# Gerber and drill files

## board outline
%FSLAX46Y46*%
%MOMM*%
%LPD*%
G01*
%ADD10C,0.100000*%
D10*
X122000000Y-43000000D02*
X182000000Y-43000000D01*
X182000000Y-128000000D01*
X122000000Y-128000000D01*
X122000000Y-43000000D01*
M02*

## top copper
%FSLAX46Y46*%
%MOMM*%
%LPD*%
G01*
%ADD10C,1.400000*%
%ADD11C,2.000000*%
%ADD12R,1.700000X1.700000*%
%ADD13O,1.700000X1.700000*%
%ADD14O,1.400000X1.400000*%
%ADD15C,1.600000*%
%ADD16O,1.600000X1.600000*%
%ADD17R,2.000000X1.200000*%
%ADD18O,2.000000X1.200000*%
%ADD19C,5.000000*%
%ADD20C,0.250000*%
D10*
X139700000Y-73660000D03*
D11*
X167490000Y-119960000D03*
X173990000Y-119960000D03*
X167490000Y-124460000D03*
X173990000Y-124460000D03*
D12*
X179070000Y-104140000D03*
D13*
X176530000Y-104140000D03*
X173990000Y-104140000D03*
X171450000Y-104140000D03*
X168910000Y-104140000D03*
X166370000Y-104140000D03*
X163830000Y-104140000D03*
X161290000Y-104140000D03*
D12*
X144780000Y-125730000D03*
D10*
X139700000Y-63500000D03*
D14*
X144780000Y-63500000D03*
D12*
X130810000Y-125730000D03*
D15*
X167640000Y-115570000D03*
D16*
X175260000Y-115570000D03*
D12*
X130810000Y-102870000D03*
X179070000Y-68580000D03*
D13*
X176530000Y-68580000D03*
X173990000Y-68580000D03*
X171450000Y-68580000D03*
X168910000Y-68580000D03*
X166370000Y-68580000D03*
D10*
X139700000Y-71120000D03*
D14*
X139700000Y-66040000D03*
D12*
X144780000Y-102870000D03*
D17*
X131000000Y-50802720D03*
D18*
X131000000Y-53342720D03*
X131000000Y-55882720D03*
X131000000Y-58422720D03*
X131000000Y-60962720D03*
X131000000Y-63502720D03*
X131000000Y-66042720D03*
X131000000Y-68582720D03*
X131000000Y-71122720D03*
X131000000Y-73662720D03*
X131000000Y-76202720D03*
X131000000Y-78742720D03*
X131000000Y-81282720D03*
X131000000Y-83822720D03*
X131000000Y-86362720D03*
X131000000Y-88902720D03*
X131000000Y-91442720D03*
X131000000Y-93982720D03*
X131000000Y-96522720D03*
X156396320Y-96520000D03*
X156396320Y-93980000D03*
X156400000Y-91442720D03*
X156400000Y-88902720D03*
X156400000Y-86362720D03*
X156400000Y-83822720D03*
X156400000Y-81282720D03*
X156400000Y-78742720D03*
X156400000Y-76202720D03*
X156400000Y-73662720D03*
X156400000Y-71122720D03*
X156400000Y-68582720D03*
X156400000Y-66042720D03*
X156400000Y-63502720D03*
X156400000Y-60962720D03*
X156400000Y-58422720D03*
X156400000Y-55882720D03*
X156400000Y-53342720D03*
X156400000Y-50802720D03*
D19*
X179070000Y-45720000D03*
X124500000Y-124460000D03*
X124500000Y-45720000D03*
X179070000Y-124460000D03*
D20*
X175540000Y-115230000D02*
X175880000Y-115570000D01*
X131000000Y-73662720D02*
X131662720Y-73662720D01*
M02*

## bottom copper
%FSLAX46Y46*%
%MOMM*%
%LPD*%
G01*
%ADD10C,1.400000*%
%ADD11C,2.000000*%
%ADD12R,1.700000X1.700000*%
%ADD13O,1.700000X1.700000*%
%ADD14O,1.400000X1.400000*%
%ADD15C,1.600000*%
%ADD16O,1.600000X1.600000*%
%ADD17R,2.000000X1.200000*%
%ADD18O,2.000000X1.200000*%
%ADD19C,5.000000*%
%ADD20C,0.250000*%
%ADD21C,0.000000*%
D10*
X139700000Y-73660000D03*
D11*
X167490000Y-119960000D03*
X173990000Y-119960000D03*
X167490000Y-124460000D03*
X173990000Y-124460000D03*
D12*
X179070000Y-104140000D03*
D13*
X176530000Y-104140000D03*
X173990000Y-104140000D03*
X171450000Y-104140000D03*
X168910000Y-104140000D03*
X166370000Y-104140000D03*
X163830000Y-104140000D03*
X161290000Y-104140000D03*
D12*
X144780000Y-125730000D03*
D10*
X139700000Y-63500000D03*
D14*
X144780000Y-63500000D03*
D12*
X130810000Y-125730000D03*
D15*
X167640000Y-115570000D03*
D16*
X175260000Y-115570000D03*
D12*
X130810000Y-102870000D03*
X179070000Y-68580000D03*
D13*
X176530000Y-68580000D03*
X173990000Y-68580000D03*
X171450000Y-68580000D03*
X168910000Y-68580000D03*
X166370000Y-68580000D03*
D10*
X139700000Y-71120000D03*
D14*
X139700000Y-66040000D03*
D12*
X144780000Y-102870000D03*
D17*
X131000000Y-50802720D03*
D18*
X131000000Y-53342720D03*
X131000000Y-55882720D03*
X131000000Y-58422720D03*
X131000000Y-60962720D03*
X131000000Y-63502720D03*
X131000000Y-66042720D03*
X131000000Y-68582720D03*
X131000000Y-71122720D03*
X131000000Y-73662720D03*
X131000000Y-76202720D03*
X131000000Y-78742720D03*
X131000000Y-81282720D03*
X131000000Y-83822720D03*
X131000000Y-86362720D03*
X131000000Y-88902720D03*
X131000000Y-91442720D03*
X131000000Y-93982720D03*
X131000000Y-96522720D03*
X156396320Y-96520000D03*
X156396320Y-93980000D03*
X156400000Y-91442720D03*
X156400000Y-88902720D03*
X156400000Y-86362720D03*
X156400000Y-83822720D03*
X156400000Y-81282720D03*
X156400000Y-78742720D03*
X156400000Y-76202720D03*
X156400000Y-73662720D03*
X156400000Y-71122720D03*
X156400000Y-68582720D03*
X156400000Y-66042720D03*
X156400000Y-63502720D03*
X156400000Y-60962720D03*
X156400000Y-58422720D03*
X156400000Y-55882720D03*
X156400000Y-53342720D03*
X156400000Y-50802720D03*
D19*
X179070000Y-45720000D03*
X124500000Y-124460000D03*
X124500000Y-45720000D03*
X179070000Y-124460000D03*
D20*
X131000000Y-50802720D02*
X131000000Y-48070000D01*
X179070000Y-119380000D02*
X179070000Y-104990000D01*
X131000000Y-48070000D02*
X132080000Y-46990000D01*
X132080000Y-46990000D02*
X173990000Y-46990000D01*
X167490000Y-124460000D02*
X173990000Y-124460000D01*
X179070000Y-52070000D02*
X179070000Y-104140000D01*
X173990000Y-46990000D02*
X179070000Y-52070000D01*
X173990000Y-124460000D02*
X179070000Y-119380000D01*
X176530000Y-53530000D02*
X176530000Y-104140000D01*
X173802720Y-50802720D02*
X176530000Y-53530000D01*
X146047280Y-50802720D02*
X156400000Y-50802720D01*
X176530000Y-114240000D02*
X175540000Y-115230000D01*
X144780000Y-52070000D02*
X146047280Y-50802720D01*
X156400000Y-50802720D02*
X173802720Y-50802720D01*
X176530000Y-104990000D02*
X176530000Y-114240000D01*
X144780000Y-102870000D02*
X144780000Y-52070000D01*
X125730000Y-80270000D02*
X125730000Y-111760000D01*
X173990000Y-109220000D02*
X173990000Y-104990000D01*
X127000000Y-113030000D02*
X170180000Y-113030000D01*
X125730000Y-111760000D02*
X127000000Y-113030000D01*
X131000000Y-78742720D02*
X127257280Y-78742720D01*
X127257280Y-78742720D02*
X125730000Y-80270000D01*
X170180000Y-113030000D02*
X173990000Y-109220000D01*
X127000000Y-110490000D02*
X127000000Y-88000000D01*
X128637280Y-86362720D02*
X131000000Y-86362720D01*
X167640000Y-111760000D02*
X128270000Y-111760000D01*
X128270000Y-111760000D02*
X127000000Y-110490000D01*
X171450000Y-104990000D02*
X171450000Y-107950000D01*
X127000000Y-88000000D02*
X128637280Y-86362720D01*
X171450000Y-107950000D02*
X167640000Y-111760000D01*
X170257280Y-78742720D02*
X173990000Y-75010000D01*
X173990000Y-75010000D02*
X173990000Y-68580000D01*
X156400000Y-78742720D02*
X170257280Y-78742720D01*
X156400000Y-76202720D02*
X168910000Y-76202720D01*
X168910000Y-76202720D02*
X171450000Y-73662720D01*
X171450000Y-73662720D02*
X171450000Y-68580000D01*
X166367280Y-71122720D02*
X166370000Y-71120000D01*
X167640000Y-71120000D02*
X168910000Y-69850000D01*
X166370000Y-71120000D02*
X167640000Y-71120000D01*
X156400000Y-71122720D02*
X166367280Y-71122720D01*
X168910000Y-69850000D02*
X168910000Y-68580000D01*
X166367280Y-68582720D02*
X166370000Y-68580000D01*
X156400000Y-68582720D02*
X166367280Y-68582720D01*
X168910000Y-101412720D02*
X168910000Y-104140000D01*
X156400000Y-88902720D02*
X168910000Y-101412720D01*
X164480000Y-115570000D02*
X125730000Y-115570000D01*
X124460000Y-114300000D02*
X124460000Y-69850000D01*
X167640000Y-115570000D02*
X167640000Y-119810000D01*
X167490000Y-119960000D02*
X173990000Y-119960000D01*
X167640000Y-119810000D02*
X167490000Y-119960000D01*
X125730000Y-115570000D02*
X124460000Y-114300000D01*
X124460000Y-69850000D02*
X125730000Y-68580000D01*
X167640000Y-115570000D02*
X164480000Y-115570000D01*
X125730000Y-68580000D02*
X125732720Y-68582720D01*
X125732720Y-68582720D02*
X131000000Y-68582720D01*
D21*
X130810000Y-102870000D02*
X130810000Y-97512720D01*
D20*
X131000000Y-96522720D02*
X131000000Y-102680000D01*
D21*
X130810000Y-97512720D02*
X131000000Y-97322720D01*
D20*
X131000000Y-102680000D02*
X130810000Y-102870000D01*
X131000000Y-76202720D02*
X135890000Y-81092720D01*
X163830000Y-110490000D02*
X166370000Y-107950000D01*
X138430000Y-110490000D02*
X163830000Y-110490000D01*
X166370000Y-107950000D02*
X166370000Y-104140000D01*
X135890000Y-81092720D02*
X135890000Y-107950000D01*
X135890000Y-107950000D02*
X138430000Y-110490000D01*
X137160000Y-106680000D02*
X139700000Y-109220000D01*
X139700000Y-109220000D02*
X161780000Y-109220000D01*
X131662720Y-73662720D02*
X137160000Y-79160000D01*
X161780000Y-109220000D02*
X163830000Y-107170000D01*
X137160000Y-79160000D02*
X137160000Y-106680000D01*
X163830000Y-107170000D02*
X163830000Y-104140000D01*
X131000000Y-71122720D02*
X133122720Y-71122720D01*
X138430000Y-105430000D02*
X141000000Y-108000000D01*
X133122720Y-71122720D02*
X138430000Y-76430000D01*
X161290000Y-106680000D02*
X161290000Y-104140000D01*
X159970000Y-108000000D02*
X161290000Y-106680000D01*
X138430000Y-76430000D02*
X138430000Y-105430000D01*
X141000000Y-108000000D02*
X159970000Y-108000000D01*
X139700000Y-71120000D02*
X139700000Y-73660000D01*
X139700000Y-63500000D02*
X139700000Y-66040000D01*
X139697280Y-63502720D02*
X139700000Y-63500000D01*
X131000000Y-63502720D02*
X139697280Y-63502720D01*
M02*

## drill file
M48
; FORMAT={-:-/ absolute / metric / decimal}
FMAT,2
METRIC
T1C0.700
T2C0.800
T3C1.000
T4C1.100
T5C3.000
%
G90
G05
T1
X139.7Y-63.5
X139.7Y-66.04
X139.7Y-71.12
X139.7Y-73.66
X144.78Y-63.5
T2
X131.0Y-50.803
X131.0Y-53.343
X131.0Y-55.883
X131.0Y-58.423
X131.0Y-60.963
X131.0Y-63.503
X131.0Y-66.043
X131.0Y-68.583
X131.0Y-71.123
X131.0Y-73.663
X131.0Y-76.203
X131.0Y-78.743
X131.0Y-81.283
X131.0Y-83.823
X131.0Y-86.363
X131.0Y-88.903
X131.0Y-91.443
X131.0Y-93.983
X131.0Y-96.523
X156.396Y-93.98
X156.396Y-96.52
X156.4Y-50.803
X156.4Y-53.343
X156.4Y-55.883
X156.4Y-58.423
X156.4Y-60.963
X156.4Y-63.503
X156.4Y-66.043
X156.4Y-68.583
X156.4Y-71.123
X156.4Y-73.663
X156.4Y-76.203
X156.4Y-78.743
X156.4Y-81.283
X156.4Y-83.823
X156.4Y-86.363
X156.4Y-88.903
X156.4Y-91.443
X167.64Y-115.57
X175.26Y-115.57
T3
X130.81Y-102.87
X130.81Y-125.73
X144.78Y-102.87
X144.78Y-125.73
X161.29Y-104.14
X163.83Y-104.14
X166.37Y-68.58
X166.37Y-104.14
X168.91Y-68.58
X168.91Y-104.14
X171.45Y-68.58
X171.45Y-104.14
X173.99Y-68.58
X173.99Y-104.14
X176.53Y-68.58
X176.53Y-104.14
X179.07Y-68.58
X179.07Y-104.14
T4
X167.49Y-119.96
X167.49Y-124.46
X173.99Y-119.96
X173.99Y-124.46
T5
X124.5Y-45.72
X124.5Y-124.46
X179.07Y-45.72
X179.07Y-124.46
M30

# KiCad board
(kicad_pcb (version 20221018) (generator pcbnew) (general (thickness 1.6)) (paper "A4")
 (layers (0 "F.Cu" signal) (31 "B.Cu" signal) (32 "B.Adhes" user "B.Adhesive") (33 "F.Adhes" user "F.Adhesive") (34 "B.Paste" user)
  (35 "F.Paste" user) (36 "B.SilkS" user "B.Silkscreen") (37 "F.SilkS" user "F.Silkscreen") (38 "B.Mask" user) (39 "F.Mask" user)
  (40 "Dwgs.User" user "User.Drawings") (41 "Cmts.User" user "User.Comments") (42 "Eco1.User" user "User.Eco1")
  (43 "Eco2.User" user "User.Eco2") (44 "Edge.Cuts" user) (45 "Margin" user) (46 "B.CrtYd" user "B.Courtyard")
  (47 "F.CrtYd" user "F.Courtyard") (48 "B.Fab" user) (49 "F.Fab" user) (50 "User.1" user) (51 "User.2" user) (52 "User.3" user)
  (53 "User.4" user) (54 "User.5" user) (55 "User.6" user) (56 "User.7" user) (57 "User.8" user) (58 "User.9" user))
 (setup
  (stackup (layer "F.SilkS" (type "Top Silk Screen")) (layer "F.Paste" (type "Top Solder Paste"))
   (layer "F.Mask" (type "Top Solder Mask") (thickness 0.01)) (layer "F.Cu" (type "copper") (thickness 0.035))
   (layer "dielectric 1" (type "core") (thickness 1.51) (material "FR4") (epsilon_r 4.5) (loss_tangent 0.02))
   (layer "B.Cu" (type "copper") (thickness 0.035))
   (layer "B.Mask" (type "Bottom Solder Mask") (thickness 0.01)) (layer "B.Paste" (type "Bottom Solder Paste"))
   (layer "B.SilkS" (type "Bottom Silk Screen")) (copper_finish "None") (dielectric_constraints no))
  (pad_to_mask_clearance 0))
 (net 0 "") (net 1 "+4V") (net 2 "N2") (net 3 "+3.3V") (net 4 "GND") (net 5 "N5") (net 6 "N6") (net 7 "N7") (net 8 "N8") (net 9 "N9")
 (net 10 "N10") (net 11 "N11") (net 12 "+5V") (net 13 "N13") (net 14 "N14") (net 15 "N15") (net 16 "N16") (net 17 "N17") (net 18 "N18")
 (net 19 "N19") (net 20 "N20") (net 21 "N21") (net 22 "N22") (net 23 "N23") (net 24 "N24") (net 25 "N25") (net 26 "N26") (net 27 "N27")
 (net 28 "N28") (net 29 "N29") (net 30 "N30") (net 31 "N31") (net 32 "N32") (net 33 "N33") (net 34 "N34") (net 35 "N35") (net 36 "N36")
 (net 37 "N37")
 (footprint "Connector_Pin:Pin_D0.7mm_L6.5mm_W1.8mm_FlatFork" (layer "F.Cu") (at 139.7 73.66 90)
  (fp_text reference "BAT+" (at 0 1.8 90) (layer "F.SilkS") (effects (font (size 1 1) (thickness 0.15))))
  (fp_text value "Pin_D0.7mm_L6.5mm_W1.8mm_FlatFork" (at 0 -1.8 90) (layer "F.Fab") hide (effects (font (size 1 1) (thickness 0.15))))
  (pad "1" thru_hole circle (at 0 0 90) (size 1.4 1.4) (drill 0.7) (layers "*.Cu" "*.Mask") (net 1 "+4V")))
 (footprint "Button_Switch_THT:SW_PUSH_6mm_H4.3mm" (layer "F.Cu") (at 167.49 119.96)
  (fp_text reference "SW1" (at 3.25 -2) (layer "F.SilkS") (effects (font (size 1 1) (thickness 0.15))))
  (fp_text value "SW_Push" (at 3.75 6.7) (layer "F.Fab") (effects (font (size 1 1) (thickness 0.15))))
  (pad "1" thru_hole circle (at 0 0 90) (size 2 2) (drill 1.1) (layers "*.Cu" "*.Mask") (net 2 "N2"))
  (pad "1" thru_hole circle (at 6.5 0 90) (size 2 2) (drill 1.1) (layers "*.Cu" "*.Mask") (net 2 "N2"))
  (pad "2" thru_hole circle (at 0 4.5 90) (size 2 2) (drill 1.1) (layers "*.Cu" "*.Mask") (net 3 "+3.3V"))
  (pad "2" thru_hole circle (at 6.5 4.5 90) (size 2 2) (drill 1.1) (layers "*.Cu" "*.Mask") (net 3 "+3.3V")))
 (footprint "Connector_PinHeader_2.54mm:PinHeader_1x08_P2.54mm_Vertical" (layer "F.Cu") (at 179.07 104.14 -90)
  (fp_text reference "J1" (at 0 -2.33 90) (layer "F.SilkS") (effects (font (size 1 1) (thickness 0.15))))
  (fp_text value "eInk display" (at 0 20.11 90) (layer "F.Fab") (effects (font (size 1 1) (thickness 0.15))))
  (pad "1" thru_hole rect (at 0 0 270) (size 1.7 1.7) (drill 1) (layers "*.Cu" "*.Mask") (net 3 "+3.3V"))
  (pad "2" thru_hole oval (at 0 2.54 270) (size 1.7 1.7) (drill 1) (layers "*.Cu" "*.Mask") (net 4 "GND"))
  (pad "3" thru_hole oval (at 0 5.08 270) (size 1.7 1.7) (drill 1) (layers "*.Cu" "*.Mask") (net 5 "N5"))
  (pad "4" thru_hole oval (at 0 7.62 270) (size 1.7 1.7) (drill 1) (layers "*.Cu" "*.Mask") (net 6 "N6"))
  (pad "5" thru_hole oval (at 0 10.16 270) (size 1.7 1.7) (drill 1) (layers "*.Cu" "*.Mask") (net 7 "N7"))
  (pad "6" thru_hole oval (at 0 12.7 270) (size 1.7 1.7) (drill 1) (layers "*.Cu" "*.Mask") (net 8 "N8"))
  (pad "7" thru_hole oval (at 0 15.24 270) (size 1.7 1.7) (drill 1) (layers "*.Cu" "*.Mask") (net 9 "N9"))
  (pad "8" thru_hole oval (at 0 17.78 270) (size 1.7 1.7) (drill 1) (layers "*.Cu" "*.Mask") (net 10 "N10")))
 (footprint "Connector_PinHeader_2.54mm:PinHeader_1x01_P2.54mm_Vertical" (layer "F.Cu") (at 144.78 125.73)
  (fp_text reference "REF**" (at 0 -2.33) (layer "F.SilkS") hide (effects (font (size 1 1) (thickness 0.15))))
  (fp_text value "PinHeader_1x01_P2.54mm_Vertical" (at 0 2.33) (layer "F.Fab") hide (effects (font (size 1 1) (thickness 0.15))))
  (pad "1" thru_hole rect (at 0 0) (size 1.7 1.7) (drill 1) (layers "*.Cu" "*.Mask")))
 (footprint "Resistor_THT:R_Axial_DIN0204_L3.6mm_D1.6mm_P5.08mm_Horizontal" (layer "F.Cu") (at 139.7 63.5)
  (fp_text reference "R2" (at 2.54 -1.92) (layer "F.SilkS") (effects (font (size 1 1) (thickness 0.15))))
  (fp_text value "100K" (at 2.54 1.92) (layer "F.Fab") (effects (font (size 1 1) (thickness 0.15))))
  (pad "1" thru_hole circle (at 0 0) (size 1.4 1.4) (drill 0.7) (layers "*.Cu" "*.Mask") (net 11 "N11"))
  (pad "2" thru_hole oval (at 5.08 0) (size 1.4 1.4) (drill 0.7) (layers "*.Cu" "*.Mask") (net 4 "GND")))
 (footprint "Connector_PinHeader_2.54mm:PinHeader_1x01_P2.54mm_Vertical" (layer "F.Cu") (at 130.81 125.73)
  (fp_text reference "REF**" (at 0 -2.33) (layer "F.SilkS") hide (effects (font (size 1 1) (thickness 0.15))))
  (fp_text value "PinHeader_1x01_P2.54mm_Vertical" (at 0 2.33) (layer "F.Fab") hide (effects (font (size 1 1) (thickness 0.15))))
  (pad "1" thru_hole rect (at 0 0) (size 1.7 1.7) (drill 1) (layers "*.Cu" "*.Mask")))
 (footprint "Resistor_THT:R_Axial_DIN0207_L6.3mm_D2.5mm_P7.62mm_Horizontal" (layer "F.Cu") (at 167.64 115.57)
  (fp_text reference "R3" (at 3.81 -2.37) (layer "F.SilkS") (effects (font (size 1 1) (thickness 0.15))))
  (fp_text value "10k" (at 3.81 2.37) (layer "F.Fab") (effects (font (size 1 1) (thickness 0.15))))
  (pad "1" thru_hole circle (at 0 0) (size 1.6 1.6) (drill 0.8) (layers "*.Cu" "*.Mask") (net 2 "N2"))
  (pad "2" thru_hole oval (at 7.62 0) (size 1.6 1.6) (drill 0.8) (layers "*.Cu" "*.Mask") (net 4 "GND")))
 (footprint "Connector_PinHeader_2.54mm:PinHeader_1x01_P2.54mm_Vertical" (layer "F.Cu") (at 130.81 102.87)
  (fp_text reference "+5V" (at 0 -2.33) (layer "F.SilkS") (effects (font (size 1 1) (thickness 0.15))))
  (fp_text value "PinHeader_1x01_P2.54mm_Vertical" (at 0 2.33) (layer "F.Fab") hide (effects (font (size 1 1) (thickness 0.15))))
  (pad "1" thru_hole rect (at 0 0) (size 1.7 1.7) (drill 1) (layers "*.Cu" "*.Mask") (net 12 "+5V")))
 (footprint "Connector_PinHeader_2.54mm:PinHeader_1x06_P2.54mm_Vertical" (layer "F.Cu") (at 179.07 68.58 -90)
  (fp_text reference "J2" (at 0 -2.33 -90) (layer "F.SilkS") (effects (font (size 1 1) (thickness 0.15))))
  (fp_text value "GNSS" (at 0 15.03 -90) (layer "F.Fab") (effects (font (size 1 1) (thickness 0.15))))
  (pad "1" thru_hole rect (at 0 0 270) (size 1.7 1.7) (drill 1) (layers "*.Cu" "*.Mask") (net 3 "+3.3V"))
  (pad "2" thru_hole oval (at 0 2.54 270) (size 1.7 1.7) (drill 1) (layers "*.Cu" "*.Mask") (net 4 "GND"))
  (pad "3" thru_hole oval (at 0 5.08 270) (size 1.7 1.7) (drill 1) (layers "*.Cu" "*.Mask") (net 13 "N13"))
  (pad "4" thru_hole oval (at 0 7.62 270) (size 1.7 1.7) (drill 1) (layers "*.Cu" "*.Mask") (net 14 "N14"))
  (pad "5" thru_hole oval (at 0 10.16 270) (size 1.7 1.7) (drill 1) (layers "*.Cu" "*.Mask") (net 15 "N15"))
  (pad "6" thru_hole oval (at 0 12.7 270) (size 1.7 1.7) (drill 1) (layers "*.Cu" "*.Mask") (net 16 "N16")))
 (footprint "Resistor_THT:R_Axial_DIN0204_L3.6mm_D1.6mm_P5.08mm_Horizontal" (layer "F.Cu") (at 139.7 71.12 90)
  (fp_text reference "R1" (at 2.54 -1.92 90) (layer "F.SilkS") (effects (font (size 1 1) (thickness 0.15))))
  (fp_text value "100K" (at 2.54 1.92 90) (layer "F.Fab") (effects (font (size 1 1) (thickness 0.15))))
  (pad "1" thru_hole circle (at 0 0 90) (size 1.4 1.4) (drill 0.7) (layers "*.Cu" "*.Mask") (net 1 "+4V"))
  (pad "2" thru_hole oval (at 5.08 0 90) (size 1.4 1.4) (drill 0.7) (layers "*.Cu" "*.Mask") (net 11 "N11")))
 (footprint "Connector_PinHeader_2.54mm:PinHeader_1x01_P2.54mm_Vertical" (layer "F.Cu") (at 144.78 102.87)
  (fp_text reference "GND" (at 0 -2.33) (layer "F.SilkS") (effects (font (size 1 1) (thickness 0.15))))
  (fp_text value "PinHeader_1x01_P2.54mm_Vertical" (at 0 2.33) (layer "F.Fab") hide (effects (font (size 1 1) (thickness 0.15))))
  (pad "1" thru_hole rect (at 0 0) (size 1.7 1.7) (drill 1) (layers "*.Cu" "*.Mask") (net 4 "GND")))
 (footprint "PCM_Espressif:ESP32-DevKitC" (layer "F.Cu") (at 131 50.80272)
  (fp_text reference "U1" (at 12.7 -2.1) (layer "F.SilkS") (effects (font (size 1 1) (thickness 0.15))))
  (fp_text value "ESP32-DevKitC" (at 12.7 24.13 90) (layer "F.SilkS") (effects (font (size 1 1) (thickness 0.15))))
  (pad "1" thru_hole rect (at 0 0 270) (size 1.2 2) (drill 0.8) (layers "*.Cu" "*.Mask") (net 3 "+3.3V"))
  (pad "2" thru_hole oval (at 0 2.54 270) (size 1.2 2) (drill 0.8) (layers "*.Cu" "*.Mask") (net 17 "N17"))
  (pad "3" thru_hole oval (at 0 5.08 270) (size 1.2 2) (drill 0.8) (layers "*.Cu" "*.Mask") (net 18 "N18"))
  (pad "4" thru_hole oval (at 0 7.62 270) (size 1.2 2) (drill 0.8) (layers "*.Cu" "*.Mask") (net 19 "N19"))
  (pad "5" thru_hole oval (at 0 10.16 270) (size 1.2 2) (drill 0.8) (layers "*.Cu" "*.Mask") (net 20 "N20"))
  (pad "6" thru_hole oval (at 0 12.7 270) (size 1.2 2) (drill 0.8) (layers "*.Cu" "*.Mask") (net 11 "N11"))
  (pad "7" thru_hole oval (at 0 15.24 270) (size 1.2 2) (drill 0.8) (layers "*.Cu" "*.Mask") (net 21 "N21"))
  (pad "8" thru_hole oval (at 0 17.78 270) (size 1.2 2) (drill 0.8) (layers "*.Cu" "*.Mask") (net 2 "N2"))
  (pad "9" thru_hole oval (at 0 20.32 270) (size 1.2 2) (drill 0.8) (layers "*.Cu" "*.Mask") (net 10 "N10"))
  (pad "10" thru_hole oval (at 0 22.86 270) (size 1.2 2) (drill 0.8) (layers "*.Cu" "*.Mask") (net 9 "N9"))
  (pad "11" thru_hole oval (at 0 25.4 270) (size 1.2 2) (drill 0.8) (layers "*.Cu" "*.Mask") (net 8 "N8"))
  (pad "12" thru_hole oval (at 0 27.94 270) (size 1.2 2) (drill 0.8) (layers "*.Cu" "*.Mask") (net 5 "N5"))
  (pad "13" thru_hole oval (at 0 30.48 270) (size 1.2 2) (drill 0.8) (layers "*.Cu" "*.Mask") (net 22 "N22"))
  (pad "14" thru_hole oval (at 0 33.02 270) (size 1.2 2) (drill 0.8) (layers "*.Cu" "*.Mask") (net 4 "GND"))
  (pad "15" thru_hole oval (at 0 35.56 270) (size 1.2 2) (drill 0.8) (layers "*.Cu" "*.Mask") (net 6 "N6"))
  (pad "16" thru_hole oval (at 0 38.1 270) (size 1.2 2) (drill 0.8) (layers "*.Cu" "*.Mask") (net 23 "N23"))
  (pad "17" thru_hole oval (at 0 40.64 270) (size 1.2 2) (drill 0.8) (layers "*.Cu" "*.Mask") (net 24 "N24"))
  (pad "18" thru_hole oval (at 0 43.18 270) (size 1.2 2) (drill 0.8) (layers "*.Cu" "*.Mask") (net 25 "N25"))
  (pad "19" thru_hole oval (at 0 45.72 270) (size 1.2 2) (drill 0.8) (layers "*.Cu" "*.Mask") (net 12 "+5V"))
  (pad "20" thru_hole oval (at 25.39632 45.71728 270) (size 1.2 2) (drill 0.8) (layers "*.Cu" "*.Mask") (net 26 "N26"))
  (pad "21" thru_hole oval (at 25.39632 43.17728 270) (size 1.2 2) (drill 0.8) (layers "*.Cu" "*.Mask") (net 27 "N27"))
  (pad "22" thru_hole oval (at 25.4 40.64 270) (size 1.2 2) (drill 0.8) (layers "*.Cu" "*.Mask") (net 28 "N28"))
  (pad "23" thru_hole oval (at 25.4 38.1 270) (size 1.2 2) (drill 0.8) (layers "*.Cu" "*.Mask") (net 7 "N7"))
  (pad "24" thru_hole oval (at 25.4 35.56 270) (size 1.2 2) (drill 0.8) (layers "*.Cu" "*.Mask") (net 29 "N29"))
  (pad "25" thru_hole oval (at 25.4 33.02 270) (size 1.2 2) (drill 0.8) (layers "*.Cu" "*.Mask") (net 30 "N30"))
  (pad "26" thru_hole oval (at 25.4 30.48 270) (size 1.2 2) (drill 0.8) (layers "*.Cu" "*.Mask") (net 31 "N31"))
  (pad "27" thru_hole oval (at 25.4 27.94 270) (size 1.2 2) (drill 0.8) (layers "*.Cu" "*.Mask") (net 13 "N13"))
  (pad "28" thru_hole oval (at 25.4 25.4 270) (size 1.2 2) (drill 0.8) (layers "*.Cu" "*.Mask") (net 14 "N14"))
  (pad "29" thru_hole oval (at 25.4 22.86 270) (size 1.2 2) (drill 0.8) (layers "*.Cu" "*.Mask") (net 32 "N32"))
  (pad "30" thru_hole oval (at 25.4 20.32 270) (size 1.2 2) (drill 0.8) (layers "*.Cu" "*.Mask") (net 15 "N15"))
  (pad "31" thru_hole oval (at 25.4 17.78 270) (size 1.2 2) (drill 0.8) (layers "*.Cu" "*.Mask") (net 16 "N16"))
  (pad "32" thru_hole oval (at 25.4 15.24 270) (size 1.2 2) (drill 0.8) (layers "*.Cu" "*.Mask") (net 4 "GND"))
  (pad "33" thru_hole oval (at 25.4 12.7 270) (size 1.2 2) (drill 0.8) (layers "*.Cu" "*.Mask") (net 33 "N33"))
  (pad "34" thru_hole oval (at 25.4 10.16 270) (size 1.2 2) (drill 0.8) (layers "*.Cu" "*.Mask") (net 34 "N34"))
  (pad "35" thru_hole oval (at 25.4 7.62 270) (size 1.2 2) (drill 0.8) (layers "*.Cu" "*.Mask") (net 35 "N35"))
  (pad "36" thru_hole oval (at 25.4 5.08 270) (size 1.2 2) (drill 0.8) (layers "*.Cu" "*.Mask") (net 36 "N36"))
  (pad "37" thru_hole oval (at 25.4 2.54 270) (size 1.2 2) (drill 0.8) (layers "*.Cu" "*.Mask") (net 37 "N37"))
  (pad "38" thru_hole oval (at 25.4 0 270) (size 1.2 2) (drill 0.8) (layers "*.Cu" "*.Mask") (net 4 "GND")))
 (gr_rect (start 122 43) (end 182 128) (stroke (width 0.1) (type default)) (fill none) (layer "Edge.Cuts"))
 (via (at 179.07 45.72) (size 5) (drill 3) (layers "F.Cu" "B.Cu") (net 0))
 (via (at 124.5 124.46) (size 5) (drill 3) (layers "F.Cu" "B.Cu") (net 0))
 (via (at 124.5 45.72) (size 5) (drill 3) (layers "F.Cu" "B.Cu") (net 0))
 (via (at 179.07 124.46) (size 5) (drill 3) (layers "F.Cu" "B.Cu") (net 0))
 (segment (start 131 50.80272) (end 131 48.07) (width 0.25) (layer "B.Cu") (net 3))
 (segment (start 179.07 119.38) (end 179.07 104.99) (width 0.25) (layer "B.Cu") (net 3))
 (segment (start 131 48.07) (end 132.08 46.99) (width 0.25) (layer "B.Cu") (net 3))
 (segment (start 132.08 46.99) (end 173.99 46.99) (width 0.25) (layer "B.Cu") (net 3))
 (segment (start 167.49 124.46) (end 173.99 124.46) (width 0.25) (layer "B.Cu") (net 3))
 (segment (start 179.07 52.07) (end 179.07 104.14) (width 0.25) (layer "B.Cu") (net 3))
 (segment (start 173.99 46.99) (end 179.07 52.07) (width 0.25) (layer "B.Cu") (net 3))
 (segment (start 173.99 124.46) (end 179.07 119.38) (width 0.25) (layer "B.Cu") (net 3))
 (segment (start 175.54 115.23) (end 175.88 115.57) (width 0.25) (layer "F.Cu") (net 4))
 (segment (start 176.53 53.53) (end 176.53 104.14) (width 0.25) (layer "B.Cu") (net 4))
 (segment (start 173.80272 50.80272) (end 176.53 53.53) (width 0.25) (layer "B.Cu") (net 4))
 (segment (start 146.04728 50.80272) (end 156.4 50.80272) (width 0.25) (layer "B.Cu") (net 4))
 (segment (start 176.53 114.24) (end 175.54 115.23) (width 0.25) (layer "B.Cu") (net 4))
 (segment (start 144.78 52.07) (end 146.04728 50.80272) (width 0.25) (layer "B.Cu") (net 4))
 (segment (start 156.4 50.80272) (end 173.80272 50.80272) (width 0.25) (layer "B.Cu") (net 4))
 (segment (start 176.53 104.99) (end 176.53 114.24) (width 0.25) (layer "B.Cu") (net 4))
 (segment (start 144.78 102.87) (end 144.78 52.07) (width 0.25) (layer "B.Cu") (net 4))
 (segment (start 125.73 80.27) (end 125.73 111.76) (width 0.25) (layer "B.Cu") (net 5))
 (segment (start 173.99 109.22) (end 173.99 104.99) (width 0.25) (layer "B.Cu") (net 5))
 (segment (start 127 113.03) (end 170.18 113.03) (width 0.25) (layer "B.Cu") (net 5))
 (segment (start 125.73 111.76) (end 127 113.03) (width 0.25) (layer "B.Cu") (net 5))
 (segment (start 131 78.74272) (end 127.25728 78.74272) (width 0.25) (layer "B.Cu") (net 5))
 (segment (start 127.25728 78.74272) (end 125.73 80.27) (width 0.25) (layer "B.Cu") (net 5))
 (segment (start 170.18 113.03) (end 173.99 109.22) (width 0.25) (layer "B.Cu") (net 5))
 (segment (start 127 110.49) (end 127 88) (width 0.25) (layer "B.Cu") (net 6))
 (segment (start 128.63728 86.36272) (end 131 86.36272) (width 0.25) (layer "B.Cu") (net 6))
 (segment (start 167.64 111.76) (end 128.27 111.76) (width 0.25) (layer "B.Cu") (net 6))
 (segment (start 128.27 111.76) (end 127 110.49) (width 0.25) (layer "B.Cu") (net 6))
 (segment (start 171.45 104.99) (end 171.45 107.95) (width 0.25) (layer "B.Cu") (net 6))
 (segment (start 127 88) (end 128.63728 86.36272) (width 0.25) (layer "B.Cu") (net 6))
 (segment (start 171.45 107.95) (end 167.64 111.76) (width 0.25) (layer "B.Cu") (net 6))
 (segment (start 170.25728 78.74272) (end 173.99 75.01) (width 0.25) (layer "B.Cu") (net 13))
 (segment (start 173.99 75.01) (end 173.99 68.58) (width 0.25) (layer "B.Cu") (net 13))
 (segment (start 156.4 78.74272) (end 170.25728 78.74272) (width 0.25) (layer "B.Cu") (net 13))
 (segment (start 156.4 76.20272) (end 168.91 76.20272) (width 0.25) (layer "B.Cu") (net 14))
 (segment (start 168.91 76.20272) (end 171.45 73.66272) (width 0.25) (layer "B.Cu") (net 14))
 (segment (start 171.45 73.66272) (end 171.45 68.58) (width 0.25) (layer "B.Cu") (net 14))
 (segment (start 166.36728 71.12272) (end 166.37 71.12) (width 0.25) (layer "B.Cu") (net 15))
 (segment (start 167.64 71.12) (end 168.91 69.85) (width 0.25) (layer "B.Cu") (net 15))
 (segment (start 166.37 71.12) (end 167.64 71.12) (width 0.25) (layer "B.Cu") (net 15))
 (segment (start 156.4 71.12272) (end 166.36728 71.12272) (width 0.25) (layer "B.Cu") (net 15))
 (segment (start 168.91 69.85) (end 168.91 68.58) (width 0.25) (layer "B.Cu") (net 15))
 (segment (start 166.36728 68.58272) (end 166.37 68.58) (width 0.25) (layer "B.Cu") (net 16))
 (segment (start 156.4 68.58272) (end 166.36728 68.58272) (width 0.25) (layer "B.Cu") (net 16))
 (segment (start 168.91 101.41272) (end 168.91 104.14) (width 0.25) (layer "B.Cu") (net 7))
 (segment (start 156.4 88.90272) (end 168.91 101.41272) (width 0.25) (layer "B.Cu") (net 7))
 (segment (start 164.48 115.57) (end 125.73 115.57) (width 0.25) (layer "B.Cu") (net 2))
 (segment (start 124.46 114.3) (end 124.46 69.85) (width 0.25) (layer "B.Cu") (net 2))
 (segment (start 167.64 115.57) (end 167.64 119.81) (width 0.25) (layer "B.Cu") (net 2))
 (segment (start 167.49 119.96) (end 173.99 119.96) (width 0.25) (layer "B.Cu") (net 2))
 (segment (start 167.64 119.81) (end 167.49 119.96) (width 0.25) (layer "B.Cu") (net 2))
 (segment (start 125.73 115.57) (end 124.46 114.3) (width 0.25) (layer "B.Cu") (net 2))
 (segment (start 124.46 69.85) (end 125.73 68.58) (width 0.25) (layer "B.Cu") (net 2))
 (segment (start 167.64 115.57) (end 164.48 115.57) (width 0.25) (layer "B.Cu") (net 2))
 (segment (start 125.73 68.58) (end 125.73272 68.58272) (width 0.25) (layer "B.Cu") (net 2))
 (segment (start 125.73272 68.58272) (end 131 68.58272) (width 0.25) (layer "B.Cu") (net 2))
 (segment (start 130.81 102.87) (end 130.81 97.51272) (width 0) (layer "B.Cu") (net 12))
 (segment (start 131 96.52272) (end 131 102.68) (width 0.25) (layer "B.Cu") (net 12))
 (segment (start 130.81 97.51272) (end 131 97.32272) (width 0) (layer "B.Cu") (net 12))
 (segment (start 131 102.68) (end 130.81 102.87) (width 0.25) (layer "B.Cu") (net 12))
 (segment (start 131 76.20272) (end 135.89 81.09272) (width 0.25) (layer "B.Cu") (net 8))
 (segment (start 163.83 110.49) (end 166.37 107.95) (width 0.25) (layer "B.Cu") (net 8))
 (segment (start 138.43 110.49) (end 163.83 110.49) (width 0.25) (layer "B.Cu") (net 8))
 (segment (start 166.37 107.95) (end 166.37 104.14) (width 0.25) (layer "B.Cu") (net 8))
 (segment (start 135.89 81.09272) (end 135.89 107.95) (width 0.25) (layer "B.Cu") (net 8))
 (segment (start 135.89 107.95) (end 138.43 110.49) (width 0.25) (layer "B.Cu") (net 8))
 (segment (start 131 73.66272) (end 131.66272 73.66272) (width 0.25) (layer "F.Cu") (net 9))
 (segment (start 137.16 106.68) (end 139.7 109.22) (width 0.25) (layer "B.Cu") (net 9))
 (segment (start 139.7 109.22) (end 161.78 109.22) (width 0.25) (layer "B.Cu") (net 9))
 (segment (start 131.66272 73.66272) (end 137.16 79.16) (width 0.25) (layer "B.Cu") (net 9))
 (segment (start 161.78 109.22) (end 163.83 107.17) (width 0.25) (layer "B.Cu") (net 9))
 (segment (start 137.16 79.16) (end 137.16 106.68) (width 0.25) (layer "B.Cu") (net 9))
 (segment (start 163.83 107.17) (end 163.83 104.14) (width 0.25) (layer "B.Cu") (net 9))
 (segment (start 131 71.12272) (end 133.12272 71.12272) (width 0.25) (layer "B.Cu") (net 10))
 (segment (start 138.43 105.43) (end 141 108) (width 0.25) (layer "B.Cu") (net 10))
 (segment (start 133.12272 71.12272) (end 138.43 76.43) (width 0.25) (layer "B.Cu") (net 10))
 (segment (start 161.29 106.68) (end 161.29 104.14) (width 0.25) (layer "B.Cu") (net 10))
 (segment (start 159.97 108) (end 161.29 106.68) (width 0.25) (layer "B.Cu") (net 10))
 (segment (start 138.43 76.43) (end 138.43 105.43) (width 0.25) (layer "B.Cu") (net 10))
 (segment (start 141 108) (end 159.97 108) (width 0.25) (layer "B.Cu") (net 10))
 (segment (start 139.7 71.12) (end 139.7 73.66) (width 0.25) (layer "B.Cu") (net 1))
 (segment (start 139.7 63.5) (end 139.7 66.04) (width 0.25) (layer "B.Cu") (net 11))
 (segment (start 139.69728 63.50272) (end 139.7 63.5) (width 0.25) (layer "B.Cu") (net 11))
 (segment (start 131 63.50272) (end 139.69728 63.50272) (width 0.25) (layer "B.Cu") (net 11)))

